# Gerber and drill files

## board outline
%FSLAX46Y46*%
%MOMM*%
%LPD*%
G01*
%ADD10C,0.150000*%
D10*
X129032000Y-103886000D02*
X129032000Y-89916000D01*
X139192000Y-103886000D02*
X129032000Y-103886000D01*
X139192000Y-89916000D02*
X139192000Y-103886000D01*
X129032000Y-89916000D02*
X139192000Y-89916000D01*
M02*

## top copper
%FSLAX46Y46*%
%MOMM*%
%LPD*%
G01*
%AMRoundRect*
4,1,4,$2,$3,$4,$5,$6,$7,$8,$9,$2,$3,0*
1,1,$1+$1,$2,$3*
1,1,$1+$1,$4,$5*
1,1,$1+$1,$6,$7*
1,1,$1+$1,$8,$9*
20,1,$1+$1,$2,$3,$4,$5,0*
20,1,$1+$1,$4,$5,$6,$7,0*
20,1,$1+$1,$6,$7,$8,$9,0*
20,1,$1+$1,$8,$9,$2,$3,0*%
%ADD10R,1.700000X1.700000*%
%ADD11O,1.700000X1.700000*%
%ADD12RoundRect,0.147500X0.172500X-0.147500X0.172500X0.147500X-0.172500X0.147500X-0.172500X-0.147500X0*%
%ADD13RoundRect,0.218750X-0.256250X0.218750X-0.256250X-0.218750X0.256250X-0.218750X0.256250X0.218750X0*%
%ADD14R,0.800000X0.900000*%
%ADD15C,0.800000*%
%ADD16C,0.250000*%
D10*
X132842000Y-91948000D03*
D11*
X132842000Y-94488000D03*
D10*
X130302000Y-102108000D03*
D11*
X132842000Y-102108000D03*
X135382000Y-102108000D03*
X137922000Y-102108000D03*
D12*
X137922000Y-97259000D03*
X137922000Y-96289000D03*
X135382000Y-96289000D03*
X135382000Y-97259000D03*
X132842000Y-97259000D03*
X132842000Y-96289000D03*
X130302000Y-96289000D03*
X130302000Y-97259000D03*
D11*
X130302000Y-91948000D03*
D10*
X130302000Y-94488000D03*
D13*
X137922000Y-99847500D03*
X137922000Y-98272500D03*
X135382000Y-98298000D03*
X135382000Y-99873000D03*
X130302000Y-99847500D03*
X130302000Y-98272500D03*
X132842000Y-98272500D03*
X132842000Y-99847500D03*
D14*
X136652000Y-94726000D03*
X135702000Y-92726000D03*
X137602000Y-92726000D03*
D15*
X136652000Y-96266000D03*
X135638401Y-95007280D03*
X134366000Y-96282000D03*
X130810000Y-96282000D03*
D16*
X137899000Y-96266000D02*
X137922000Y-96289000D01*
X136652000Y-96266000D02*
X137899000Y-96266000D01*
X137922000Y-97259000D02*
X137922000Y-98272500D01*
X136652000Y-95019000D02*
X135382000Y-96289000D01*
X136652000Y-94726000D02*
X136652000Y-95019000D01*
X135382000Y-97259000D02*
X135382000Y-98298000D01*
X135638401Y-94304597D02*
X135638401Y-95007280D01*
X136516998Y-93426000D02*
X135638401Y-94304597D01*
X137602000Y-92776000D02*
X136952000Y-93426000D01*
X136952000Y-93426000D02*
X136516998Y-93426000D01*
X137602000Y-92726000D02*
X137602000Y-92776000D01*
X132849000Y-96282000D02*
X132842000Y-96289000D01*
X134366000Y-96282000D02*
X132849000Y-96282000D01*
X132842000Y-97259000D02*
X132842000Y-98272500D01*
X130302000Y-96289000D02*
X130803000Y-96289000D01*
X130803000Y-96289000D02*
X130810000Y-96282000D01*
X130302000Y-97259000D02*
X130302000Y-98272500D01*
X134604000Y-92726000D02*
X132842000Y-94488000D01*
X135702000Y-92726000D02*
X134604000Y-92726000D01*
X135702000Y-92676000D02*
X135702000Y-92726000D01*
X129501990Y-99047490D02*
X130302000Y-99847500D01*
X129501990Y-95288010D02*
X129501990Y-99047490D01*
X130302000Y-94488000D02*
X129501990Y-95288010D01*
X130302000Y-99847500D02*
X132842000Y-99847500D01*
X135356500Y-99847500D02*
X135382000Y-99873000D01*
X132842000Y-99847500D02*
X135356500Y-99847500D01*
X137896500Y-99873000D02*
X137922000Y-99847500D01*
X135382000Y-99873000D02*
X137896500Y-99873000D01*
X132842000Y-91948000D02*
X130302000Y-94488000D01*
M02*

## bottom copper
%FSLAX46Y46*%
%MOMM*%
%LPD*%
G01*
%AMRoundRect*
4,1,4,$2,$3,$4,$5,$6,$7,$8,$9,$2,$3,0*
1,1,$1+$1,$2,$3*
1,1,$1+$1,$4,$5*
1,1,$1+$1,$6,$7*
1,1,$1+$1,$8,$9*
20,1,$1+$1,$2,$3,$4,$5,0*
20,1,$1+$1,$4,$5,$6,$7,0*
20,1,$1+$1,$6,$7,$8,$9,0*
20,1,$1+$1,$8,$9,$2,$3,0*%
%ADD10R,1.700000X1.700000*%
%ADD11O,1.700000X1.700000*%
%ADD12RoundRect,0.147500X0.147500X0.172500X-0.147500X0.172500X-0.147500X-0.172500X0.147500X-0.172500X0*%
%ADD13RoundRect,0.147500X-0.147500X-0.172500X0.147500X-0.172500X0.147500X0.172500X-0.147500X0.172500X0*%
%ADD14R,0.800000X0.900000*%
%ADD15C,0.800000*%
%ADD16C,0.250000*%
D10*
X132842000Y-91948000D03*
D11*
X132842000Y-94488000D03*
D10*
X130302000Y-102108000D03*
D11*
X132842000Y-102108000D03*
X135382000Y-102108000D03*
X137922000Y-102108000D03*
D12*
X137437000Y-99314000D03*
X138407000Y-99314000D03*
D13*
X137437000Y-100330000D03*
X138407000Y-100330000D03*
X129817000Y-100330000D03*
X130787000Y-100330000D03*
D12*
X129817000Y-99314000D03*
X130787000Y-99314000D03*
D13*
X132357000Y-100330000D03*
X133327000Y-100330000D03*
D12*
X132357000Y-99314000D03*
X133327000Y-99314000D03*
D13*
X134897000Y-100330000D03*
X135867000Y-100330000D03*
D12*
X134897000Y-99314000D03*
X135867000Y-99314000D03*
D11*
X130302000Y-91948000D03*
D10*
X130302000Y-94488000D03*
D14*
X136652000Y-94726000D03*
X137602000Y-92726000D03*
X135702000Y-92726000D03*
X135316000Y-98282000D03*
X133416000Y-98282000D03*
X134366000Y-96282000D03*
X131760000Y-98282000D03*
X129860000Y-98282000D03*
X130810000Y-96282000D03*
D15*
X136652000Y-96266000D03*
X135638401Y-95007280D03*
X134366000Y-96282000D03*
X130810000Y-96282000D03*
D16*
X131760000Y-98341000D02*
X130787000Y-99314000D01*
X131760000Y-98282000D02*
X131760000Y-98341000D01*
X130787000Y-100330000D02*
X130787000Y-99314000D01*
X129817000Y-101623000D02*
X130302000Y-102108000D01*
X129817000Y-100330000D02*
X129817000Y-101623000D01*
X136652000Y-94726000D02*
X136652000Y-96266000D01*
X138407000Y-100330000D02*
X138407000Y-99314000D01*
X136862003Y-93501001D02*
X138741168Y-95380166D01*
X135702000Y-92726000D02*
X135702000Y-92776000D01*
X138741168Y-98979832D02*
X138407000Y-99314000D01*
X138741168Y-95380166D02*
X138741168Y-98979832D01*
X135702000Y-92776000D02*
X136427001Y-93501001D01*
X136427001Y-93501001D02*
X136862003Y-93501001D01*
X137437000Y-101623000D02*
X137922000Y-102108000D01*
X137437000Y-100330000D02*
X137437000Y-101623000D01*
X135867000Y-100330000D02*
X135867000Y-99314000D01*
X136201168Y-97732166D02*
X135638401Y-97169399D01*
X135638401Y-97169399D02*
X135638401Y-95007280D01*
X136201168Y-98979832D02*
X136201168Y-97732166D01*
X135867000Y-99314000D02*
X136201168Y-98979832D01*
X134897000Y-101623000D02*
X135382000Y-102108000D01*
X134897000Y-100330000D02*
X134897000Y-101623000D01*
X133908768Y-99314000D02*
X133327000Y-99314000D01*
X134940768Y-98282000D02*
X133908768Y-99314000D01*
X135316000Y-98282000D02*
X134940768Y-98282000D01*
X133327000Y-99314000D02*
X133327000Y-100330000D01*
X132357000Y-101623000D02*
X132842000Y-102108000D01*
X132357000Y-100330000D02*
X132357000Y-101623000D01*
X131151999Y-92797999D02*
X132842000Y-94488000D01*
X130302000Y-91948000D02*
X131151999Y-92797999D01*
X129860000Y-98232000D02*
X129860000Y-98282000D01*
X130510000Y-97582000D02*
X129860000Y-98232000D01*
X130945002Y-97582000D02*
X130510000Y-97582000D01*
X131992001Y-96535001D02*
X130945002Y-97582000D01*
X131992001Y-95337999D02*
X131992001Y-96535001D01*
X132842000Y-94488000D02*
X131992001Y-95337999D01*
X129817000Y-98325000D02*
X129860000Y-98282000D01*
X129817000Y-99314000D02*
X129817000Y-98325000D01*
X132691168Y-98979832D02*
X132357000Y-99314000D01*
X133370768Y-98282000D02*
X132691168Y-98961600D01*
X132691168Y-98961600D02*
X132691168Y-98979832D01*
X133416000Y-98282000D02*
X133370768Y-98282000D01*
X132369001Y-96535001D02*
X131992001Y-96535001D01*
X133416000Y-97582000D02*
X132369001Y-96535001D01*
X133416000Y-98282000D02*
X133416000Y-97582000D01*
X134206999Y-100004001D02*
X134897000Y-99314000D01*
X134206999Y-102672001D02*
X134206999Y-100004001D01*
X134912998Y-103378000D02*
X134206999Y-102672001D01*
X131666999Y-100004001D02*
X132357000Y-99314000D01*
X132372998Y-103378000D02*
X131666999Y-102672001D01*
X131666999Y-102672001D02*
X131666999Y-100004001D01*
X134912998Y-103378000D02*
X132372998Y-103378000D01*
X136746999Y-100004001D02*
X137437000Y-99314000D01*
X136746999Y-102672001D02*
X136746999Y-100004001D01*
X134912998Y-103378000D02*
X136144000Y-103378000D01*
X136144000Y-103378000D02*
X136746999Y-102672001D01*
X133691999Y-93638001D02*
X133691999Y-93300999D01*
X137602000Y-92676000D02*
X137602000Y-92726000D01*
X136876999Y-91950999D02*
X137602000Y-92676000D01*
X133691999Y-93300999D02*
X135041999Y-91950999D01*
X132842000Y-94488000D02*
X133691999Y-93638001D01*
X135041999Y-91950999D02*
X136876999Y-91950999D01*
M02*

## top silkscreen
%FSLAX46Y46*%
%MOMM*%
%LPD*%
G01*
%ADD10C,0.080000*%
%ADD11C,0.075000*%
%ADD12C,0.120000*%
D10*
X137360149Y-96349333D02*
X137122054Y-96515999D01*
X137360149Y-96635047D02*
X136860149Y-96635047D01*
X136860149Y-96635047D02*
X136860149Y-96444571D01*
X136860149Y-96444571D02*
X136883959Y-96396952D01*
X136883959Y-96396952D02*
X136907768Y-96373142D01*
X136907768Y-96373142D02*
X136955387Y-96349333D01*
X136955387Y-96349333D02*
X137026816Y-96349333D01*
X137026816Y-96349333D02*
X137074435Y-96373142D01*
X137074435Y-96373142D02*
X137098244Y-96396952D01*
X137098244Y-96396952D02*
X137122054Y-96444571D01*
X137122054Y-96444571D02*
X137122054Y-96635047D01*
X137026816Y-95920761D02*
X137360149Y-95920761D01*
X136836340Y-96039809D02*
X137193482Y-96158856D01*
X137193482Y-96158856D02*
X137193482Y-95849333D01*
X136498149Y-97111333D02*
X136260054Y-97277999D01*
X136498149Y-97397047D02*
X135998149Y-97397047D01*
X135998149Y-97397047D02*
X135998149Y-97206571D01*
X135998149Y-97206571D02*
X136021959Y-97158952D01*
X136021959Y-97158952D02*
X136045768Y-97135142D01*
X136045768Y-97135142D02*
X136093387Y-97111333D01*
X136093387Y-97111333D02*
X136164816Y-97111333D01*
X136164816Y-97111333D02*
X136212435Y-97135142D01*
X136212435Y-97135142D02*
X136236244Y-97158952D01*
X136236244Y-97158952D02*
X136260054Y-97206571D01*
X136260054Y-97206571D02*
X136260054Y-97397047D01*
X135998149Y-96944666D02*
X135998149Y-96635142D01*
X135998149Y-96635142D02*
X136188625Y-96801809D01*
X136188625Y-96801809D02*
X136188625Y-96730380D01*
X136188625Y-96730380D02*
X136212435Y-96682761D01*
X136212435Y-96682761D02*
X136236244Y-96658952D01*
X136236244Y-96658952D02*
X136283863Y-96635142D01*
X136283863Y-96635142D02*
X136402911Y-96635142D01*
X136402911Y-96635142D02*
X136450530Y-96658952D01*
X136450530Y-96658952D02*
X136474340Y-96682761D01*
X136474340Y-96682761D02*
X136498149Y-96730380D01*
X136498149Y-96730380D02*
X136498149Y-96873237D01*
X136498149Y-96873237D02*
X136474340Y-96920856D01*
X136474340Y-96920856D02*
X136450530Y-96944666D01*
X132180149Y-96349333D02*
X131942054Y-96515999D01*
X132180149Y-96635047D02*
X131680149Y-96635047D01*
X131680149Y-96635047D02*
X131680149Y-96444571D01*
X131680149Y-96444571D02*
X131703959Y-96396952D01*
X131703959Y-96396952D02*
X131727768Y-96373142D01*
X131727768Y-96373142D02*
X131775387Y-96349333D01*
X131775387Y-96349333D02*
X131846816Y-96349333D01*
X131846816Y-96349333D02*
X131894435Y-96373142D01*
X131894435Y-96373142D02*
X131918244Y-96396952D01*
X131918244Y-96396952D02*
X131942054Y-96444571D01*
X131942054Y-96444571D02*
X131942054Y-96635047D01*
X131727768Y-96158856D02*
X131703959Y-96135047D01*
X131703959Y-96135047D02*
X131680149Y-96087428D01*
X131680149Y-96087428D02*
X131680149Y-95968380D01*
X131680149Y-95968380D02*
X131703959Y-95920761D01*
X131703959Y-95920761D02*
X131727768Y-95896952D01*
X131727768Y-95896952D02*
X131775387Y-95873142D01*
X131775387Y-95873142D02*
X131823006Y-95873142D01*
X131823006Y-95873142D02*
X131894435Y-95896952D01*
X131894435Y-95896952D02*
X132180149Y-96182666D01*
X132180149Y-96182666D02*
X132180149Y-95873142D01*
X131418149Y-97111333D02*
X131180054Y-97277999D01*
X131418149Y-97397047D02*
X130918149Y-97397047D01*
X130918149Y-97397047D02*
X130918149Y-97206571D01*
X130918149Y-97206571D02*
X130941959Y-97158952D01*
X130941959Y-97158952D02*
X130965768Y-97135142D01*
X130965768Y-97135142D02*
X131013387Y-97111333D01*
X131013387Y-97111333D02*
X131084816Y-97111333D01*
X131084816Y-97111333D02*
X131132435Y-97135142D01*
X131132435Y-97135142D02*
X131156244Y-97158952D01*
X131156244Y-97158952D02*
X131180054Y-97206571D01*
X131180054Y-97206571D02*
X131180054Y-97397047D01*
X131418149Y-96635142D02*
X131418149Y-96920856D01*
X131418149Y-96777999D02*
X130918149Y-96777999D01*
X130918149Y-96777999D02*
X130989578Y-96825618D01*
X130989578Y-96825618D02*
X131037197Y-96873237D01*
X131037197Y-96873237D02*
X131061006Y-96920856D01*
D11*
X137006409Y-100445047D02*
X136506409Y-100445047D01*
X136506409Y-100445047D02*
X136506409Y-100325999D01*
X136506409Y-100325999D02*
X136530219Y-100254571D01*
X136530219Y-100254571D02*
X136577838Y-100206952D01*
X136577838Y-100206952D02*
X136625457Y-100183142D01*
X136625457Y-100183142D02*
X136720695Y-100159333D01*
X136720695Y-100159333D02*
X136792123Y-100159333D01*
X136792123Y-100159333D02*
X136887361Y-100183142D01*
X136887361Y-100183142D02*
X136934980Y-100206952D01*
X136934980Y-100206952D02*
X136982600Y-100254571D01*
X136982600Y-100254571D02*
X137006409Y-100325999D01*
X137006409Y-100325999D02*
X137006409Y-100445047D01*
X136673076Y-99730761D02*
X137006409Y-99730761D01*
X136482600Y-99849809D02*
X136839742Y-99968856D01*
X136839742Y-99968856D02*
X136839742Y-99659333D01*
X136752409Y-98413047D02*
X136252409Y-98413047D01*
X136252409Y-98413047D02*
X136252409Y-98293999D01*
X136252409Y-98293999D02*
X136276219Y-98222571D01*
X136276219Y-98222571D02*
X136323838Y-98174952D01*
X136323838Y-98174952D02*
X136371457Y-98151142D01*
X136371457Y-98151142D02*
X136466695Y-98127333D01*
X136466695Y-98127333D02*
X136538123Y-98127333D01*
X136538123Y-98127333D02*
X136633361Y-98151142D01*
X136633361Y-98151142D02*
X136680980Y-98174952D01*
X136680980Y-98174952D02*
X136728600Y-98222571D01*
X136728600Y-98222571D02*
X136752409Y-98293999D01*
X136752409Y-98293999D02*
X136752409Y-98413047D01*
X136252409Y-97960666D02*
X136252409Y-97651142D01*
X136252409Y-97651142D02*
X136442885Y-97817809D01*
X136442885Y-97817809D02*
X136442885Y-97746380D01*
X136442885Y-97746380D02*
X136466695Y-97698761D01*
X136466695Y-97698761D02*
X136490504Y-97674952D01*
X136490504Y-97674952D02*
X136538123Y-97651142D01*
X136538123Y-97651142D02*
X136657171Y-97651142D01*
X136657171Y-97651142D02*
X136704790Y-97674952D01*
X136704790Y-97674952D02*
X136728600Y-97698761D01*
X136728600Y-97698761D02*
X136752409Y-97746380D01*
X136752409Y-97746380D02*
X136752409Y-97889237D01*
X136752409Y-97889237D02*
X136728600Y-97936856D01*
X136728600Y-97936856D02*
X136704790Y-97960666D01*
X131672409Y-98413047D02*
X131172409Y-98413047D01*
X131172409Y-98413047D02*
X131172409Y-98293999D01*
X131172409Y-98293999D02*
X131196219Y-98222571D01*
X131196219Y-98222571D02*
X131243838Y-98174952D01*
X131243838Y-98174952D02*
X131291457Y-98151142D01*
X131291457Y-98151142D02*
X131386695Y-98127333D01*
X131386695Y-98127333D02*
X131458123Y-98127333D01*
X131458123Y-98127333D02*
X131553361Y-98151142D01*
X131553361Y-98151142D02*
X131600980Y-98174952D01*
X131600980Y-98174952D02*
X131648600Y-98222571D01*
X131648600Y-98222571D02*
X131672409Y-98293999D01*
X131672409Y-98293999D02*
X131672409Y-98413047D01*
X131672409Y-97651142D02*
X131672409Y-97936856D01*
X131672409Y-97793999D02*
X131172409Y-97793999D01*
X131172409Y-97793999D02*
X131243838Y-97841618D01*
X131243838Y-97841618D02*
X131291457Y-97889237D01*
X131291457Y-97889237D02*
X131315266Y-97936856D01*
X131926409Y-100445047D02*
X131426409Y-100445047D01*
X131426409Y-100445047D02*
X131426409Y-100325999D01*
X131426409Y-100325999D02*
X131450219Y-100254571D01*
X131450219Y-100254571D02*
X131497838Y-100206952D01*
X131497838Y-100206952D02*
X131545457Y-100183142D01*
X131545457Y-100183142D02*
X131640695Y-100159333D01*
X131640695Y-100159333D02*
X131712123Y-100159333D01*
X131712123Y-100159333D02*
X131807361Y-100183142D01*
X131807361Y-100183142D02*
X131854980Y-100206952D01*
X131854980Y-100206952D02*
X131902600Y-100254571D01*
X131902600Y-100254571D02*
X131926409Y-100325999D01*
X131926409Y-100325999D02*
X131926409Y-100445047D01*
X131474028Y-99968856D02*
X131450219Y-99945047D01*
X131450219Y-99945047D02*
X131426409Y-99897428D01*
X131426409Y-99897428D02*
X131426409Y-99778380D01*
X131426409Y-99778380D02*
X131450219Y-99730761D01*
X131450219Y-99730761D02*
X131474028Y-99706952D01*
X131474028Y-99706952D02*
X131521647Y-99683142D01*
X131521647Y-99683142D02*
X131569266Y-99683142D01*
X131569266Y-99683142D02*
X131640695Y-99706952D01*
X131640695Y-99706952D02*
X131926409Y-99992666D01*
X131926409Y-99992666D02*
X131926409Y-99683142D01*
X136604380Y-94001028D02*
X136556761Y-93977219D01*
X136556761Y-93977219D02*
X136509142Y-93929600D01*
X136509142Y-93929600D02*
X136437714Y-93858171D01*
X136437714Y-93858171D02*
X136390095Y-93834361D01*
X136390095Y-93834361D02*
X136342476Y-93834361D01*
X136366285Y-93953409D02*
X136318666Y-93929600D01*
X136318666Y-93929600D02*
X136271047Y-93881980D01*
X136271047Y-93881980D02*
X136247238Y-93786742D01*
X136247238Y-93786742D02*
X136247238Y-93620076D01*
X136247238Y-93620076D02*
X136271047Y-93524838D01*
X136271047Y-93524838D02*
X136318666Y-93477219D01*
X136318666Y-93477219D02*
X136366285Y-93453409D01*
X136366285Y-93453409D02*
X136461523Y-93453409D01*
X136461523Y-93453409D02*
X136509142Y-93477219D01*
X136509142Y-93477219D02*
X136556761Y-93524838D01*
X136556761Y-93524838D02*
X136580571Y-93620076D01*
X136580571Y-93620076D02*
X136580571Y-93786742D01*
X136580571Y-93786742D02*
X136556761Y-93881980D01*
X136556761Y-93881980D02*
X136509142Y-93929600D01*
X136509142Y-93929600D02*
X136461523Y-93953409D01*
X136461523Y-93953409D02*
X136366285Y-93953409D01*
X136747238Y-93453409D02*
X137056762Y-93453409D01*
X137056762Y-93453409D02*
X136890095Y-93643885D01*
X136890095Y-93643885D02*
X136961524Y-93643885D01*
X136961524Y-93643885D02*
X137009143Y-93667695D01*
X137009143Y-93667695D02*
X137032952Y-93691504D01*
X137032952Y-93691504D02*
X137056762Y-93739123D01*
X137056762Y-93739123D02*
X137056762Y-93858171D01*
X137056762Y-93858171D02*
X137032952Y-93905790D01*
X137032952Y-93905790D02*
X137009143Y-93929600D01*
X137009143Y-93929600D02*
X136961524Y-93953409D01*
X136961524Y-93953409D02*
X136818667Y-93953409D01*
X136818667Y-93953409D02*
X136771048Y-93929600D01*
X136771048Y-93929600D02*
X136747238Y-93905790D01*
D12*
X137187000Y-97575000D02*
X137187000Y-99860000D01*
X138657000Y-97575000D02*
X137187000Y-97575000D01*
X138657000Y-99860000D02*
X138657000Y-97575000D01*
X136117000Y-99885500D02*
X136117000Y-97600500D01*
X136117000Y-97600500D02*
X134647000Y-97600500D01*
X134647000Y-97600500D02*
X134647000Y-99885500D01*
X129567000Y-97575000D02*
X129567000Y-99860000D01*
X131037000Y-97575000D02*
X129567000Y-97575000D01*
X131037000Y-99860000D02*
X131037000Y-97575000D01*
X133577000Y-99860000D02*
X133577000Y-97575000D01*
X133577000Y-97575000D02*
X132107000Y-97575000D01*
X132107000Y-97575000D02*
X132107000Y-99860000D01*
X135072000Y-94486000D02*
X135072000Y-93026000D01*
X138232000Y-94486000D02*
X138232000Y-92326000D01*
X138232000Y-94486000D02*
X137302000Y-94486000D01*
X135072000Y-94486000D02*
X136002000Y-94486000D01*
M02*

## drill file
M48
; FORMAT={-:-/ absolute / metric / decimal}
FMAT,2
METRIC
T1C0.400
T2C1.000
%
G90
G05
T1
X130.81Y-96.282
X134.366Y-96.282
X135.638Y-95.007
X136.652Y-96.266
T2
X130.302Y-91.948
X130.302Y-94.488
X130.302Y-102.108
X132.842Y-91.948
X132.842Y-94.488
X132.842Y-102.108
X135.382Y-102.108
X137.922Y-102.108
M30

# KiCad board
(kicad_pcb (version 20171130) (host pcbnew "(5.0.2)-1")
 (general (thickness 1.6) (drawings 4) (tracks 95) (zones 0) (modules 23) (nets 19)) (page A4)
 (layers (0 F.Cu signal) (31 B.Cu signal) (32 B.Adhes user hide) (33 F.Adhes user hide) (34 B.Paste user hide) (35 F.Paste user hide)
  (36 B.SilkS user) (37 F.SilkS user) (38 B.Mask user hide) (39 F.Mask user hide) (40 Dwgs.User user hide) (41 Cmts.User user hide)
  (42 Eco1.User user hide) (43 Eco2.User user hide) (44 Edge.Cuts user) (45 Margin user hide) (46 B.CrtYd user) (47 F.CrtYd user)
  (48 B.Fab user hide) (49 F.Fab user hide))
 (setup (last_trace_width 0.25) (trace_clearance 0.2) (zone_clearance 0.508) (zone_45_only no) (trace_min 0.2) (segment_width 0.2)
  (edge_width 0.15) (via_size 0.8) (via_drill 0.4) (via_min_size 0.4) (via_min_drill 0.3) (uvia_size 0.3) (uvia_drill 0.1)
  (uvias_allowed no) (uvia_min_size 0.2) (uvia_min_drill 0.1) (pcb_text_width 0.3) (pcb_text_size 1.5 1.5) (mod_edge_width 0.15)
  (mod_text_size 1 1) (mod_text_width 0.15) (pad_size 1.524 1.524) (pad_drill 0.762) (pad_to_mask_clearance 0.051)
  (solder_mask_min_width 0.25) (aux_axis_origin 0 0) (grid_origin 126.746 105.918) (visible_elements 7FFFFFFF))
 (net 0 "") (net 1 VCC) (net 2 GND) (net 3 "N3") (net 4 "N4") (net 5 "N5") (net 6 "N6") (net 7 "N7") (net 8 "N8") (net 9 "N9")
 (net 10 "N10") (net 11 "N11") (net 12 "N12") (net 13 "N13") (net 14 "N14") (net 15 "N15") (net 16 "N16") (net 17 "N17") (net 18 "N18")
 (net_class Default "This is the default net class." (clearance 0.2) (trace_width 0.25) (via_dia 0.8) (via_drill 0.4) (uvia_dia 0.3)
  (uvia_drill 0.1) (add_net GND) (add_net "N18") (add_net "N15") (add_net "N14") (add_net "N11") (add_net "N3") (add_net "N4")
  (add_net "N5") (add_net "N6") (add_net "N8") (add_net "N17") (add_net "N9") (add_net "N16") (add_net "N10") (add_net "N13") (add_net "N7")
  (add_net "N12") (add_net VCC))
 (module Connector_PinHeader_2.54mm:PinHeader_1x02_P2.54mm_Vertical (layer B.Cu) (at 132.842 91.948 180)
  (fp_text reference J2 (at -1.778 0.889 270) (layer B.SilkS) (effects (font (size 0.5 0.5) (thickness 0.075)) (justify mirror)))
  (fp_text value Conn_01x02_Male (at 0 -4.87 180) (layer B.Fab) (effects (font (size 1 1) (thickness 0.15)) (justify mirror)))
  (pad 1 thru_hole rect (at 0 0 180) (size 1.7 1.7) (drill 1) (layers *.Cu *.Mask) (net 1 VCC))
  (pad 2 thru_hole oval (at 0 -2.54 180) (size 1.7 1.7) (drill 1) (layers *.Cu *.Mask) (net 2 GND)))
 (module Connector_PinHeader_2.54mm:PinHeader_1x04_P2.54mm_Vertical (layer B.Cu) (at 130.302 102.108 270)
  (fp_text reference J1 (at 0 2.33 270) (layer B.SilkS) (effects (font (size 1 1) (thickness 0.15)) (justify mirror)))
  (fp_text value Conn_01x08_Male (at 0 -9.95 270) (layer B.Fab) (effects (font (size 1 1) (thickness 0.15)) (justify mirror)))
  (pad 1 thru_hole rect (at 0 0 270) (size 1.7 1.7) (drill 1) (layers *.Cu *.Mask) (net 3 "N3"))
  (pad 2 thru_hole oval (at 0 -2.54 270) (size 1.7 1.7) (drill 1) (layers *.Cu *.Mask) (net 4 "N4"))
  (pad 3 thru_hole oval (at 0 -5.08 270) (size 1.7 1.7) (drill 1) (layers *.Cu *.Mask) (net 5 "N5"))
  (pad 4 thru_hole oval (at 0 -7.62 270) (size 1.7 1.7) (drill 1) (layers *.Cu *.Mask) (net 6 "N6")))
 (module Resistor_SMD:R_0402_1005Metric (layer B.Cu) (at 137.922 99.314 180)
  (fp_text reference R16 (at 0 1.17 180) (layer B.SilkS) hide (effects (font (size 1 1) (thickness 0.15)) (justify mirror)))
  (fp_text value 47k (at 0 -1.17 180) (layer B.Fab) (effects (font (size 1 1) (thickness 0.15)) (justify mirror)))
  (pad 2 smd roundrect (at 0.485 0 180) (size 0.59 0.64) (layers B.Cu B.Paste B.Mask) (roundrect_rratio 0.25) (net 2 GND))
  (pad 1 smd roundrect (at -0.485 0 180) (size 0.59 0.64) (layers B.Cu B.Paste B.Mask) (roundrect_rratio 0.25) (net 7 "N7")))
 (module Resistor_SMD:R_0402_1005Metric (layer B.Cu) (at 137.922 100.33)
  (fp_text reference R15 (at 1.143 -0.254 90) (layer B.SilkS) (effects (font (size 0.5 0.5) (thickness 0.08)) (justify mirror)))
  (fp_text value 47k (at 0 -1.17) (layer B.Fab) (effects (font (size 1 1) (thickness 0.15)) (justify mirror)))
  (pad 1 smd roundrect (at -0.485 0) (size 0.59 0.64) (layers B.Cu B.Paste B.Mask) (roundrect_rratio 0.25) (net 6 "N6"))
  (pad 2 smd roundrect (at 0.485 0) (size 0.59 0.64) (layers B.Cu B.Paste B.Mask) (roundrect_rratio 0.25) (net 7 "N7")))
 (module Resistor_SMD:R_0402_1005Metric (layer B.Cu) (at 130.302 100.33)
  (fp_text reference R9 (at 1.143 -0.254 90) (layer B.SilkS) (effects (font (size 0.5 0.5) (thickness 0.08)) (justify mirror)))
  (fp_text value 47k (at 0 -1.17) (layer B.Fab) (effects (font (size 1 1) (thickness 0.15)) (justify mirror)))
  (pad 1 smd roundrect (at -0.485 0) (size 0.59 0.64) (layers B.Cu B.Paste B.Mask) (roundrect_rratio 0.25) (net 3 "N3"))
  (pad 2 smd roundrect (at 0.485 0) (size 0.59 0.64) (layers B.Cu B.Paste B.Mask) (roundrect_rratio 0.25) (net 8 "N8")))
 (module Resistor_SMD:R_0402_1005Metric (layer B.Cu) (at 130.302 99.314 180)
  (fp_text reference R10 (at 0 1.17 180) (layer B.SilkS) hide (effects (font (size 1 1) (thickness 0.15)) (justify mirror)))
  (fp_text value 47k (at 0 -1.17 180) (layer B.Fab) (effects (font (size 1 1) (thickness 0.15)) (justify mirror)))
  (pad 2 smd roundrect (at 0.485 0 180) (size 0.59 0.64) (layers B.Cu B.Paste B.Mask) (roundrect_rratio 0.25) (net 2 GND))
  (pad 1 smd roundrect (at -0.485 0 180) (size 0.59 0.64) (layers B.Cu B.Paste B.Mask) (roundrect_rratio 0.25) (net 8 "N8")))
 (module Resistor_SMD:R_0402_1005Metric (layer B.Cu) (at 132.842 100.33)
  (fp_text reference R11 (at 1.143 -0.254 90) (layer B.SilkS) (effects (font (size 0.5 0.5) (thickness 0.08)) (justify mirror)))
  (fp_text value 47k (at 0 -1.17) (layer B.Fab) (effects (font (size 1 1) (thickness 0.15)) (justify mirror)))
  (pad 1 smd roundrect (at -0.485 0) (size 0.59 0.64) (layers B.Cu B.Paste B.Mask) (roundrect_rratio 0.25) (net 4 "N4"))
  (pad 2 smd roundrect (at 0.485 0) (size 0.59 0.64) (layers B.Cu B.Paste B.Mask) (roundrect_rratio 0.25) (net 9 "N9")))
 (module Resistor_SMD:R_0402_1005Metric (layer B.Cu) (at 132.842 99.314 180)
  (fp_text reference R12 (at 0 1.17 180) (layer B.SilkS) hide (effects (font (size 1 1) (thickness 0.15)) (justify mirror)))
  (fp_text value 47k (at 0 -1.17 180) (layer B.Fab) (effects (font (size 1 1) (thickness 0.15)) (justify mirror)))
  (pad 2 smd roundrect (at 0.485 0 180) (size 0.59 0.64) (layers B.Cu B.Paste B.Mask) (roundrect_rratio 0.25) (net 2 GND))
  (pad 1 smd roundrect (at -0.485 0 180) (size 0.59 0.64) (layers B.Cu B.Paste B.Mask) (roundrect_rratio 0.25) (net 9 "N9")))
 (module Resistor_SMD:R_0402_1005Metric (layer B.Cu) (at 135.382 100.33)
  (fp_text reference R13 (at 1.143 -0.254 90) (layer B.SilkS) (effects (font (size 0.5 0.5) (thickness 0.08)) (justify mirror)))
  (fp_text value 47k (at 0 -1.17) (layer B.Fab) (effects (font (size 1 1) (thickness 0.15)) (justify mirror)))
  (pad 1 smd roundrect (at -0.485 0) (size 0.59 0.64) (layers B.Cu B.Paste B.Mask) (roundrect_rratio 0.25) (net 5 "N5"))
  (pad 2 smd roundrect (at 0.485 0) (size 0.59 0.64) (layers B.Cu B.Paste B.Mask) (roundrect_rratio 0.25) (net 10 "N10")))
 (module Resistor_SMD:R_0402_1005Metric (layer B.Cu) (at 135.382 99.314 180)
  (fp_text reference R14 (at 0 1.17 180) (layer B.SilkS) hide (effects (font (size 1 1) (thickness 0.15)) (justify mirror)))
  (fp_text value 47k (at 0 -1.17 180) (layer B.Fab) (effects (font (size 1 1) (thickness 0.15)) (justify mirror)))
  (pad 2 smd roundrect (at 0.485 0 180) (size 0.59 0.64) (layers B.Cu B.Paste B.Mask) (roundrect_rratio 0.25) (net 2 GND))
  (pad 1 smd roundrect (at -0.485 0 180) (size 0.59 0.64) (layers B.Cu B.Paste B.Mask) (roundrect_rratio 0.25) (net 10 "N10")))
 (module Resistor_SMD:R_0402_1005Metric (layer F.Cu) (at 137.922 96.774 90)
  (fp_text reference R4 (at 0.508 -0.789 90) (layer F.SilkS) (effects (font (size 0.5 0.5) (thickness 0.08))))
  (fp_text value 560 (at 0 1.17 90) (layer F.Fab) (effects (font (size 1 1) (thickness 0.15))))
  (pad 1 smd roundrect (at -0.485 0 90) (size 0.59 0.64) (layers F.Cu F.Paste F.Mask) (roundrect_rratio 0.25) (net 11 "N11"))
  (pad 2 smd roundrect (at 0.485 0 90) (size 0.59 0.64) (layers F.Cu F.Paste F.Mask) (roundrect_rratio 0.25) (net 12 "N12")))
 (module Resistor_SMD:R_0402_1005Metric (layer F.Cu) (at 135.382 96.774 90)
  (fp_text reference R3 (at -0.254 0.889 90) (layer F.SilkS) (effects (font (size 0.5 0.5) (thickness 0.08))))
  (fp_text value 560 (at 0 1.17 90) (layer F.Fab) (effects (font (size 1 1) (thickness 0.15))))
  (pad 2 smd roundrect (at 0.485 0 90) (size 0.59 0.64) (layers F.Cu F.Paste F.Mask) (roundrect_rratio 0.25) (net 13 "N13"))
  (pad 1 smd roundrect (at -0.485 0 90) (size 0.59 0.64) (layers F.Cu F.Paste F.Mask) (roundrect_rratio 0.25) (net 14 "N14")))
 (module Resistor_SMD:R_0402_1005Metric (layer F.Cu) (at 132.842 96.774 90)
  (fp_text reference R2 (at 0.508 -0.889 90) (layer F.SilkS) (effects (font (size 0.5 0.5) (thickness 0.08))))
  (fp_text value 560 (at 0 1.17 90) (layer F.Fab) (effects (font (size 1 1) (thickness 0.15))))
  (pad 1 smd roundrect (at -0.485 0 90) (size 0.59 0.64) (layers F.Cu F.Paste F.Mask) (roundrect_rratio 0.25) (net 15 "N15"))
  (pad 2 smd roundrect (at 0.485 0 90) (size 0.59 0.64) (layers F.Cu F.Paste F.Mask) (roundrect_rratio 0.25) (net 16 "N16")))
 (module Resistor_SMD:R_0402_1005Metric (layer F.Cu) (at 130.302 96.774 90)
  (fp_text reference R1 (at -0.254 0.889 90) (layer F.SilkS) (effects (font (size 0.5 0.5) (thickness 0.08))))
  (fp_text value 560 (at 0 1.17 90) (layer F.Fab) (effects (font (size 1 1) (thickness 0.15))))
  (pad 2 smd roundrect (at 0.485 0 90) (size 0.59 0.64) (layers F.Cu F.Paste F.Mask) (roundrect_rratio 0.25) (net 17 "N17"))
  (pad 1 smd roundrect (at -0.485 0 90) (size 0.59 0.64) (layers F.Cu F.Paste F.Mask) (roundrect_rratio 0.25) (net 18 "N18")))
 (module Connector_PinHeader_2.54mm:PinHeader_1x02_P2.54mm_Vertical (layer B.Cu) (at 130.302 94.488)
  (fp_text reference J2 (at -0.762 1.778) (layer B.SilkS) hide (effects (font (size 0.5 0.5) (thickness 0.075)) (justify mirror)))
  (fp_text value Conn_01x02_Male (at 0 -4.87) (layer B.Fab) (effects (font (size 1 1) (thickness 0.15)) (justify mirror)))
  (pad 2 thru_hole oval (at 0 -2.54) (size 1.7 1.7) (drill 1) (layers *.Cu *.Mask) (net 2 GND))
  (pad 1 thru_hole rect (at 0 0) (size 1.7 1.7) (drill 1) (layers *.Cu *.Mask) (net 1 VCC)))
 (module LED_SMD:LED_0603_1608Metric (layer F.Cu) (at 137.922 99.06 270)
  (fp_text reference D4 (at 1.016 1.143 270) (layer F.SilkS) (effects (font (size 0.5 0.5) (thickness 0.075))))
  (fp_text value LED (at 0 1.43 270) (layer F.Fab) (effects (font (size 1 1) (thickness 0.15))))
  (fp_line (start -1.485 0.735) (end 0.8 0.735) (layer F.SilkS) (width 0.12))
  (fp_line (start -1.485 -0.735) (end -1.485 0.735) (layer F.SilkS) (width 0.12))
  (fp_line (start 0.8 -0.735) (end -1.485 -0.735) (layer F.SilkS) (width 0.12))
  (pad 2 smd roundrect (at 0.7875 0 270) (size 0.875 0.95) (layers F.Cu F.Paste F.Mask) (roundrect_rratio 0.25) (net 1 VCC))
  (pad 1 smd roundrect (at -0.7875 0 270) (size 0.875 0.95) (layers F.Cu F.Paste F.Mask) (roundrect_rratio 0.25) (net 11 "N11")))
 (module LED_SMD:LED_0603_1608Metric (layer F.Cu) (at 135.382 99.0855 270)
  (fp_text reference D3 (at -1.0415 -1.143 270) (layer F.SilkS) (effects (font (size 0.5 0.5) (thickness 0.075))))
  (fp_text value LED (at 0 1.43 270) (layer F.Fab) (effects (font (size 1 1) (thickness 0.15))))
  (fp_line (start 0.8 -0.735) (end -1.485 -0.735) (layer F.SilkS) (width 0.12))
  (fp_line (start -1.485 -0.735) (end -1.485 0.735) (layer F.SilkS) (width 0.12))
  (fp_line (start -1.485 0.735) (end 0.8 0.735) (layer F.SilkS) (width 0.12))
  (pad 1 smd roundrect (at -0.7875 0 270) (size 0.875 0.95) (layers F.Cu F.Paste F.Mask) (roundrect_rratio 0.25) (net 14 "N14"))
  (pad 2 smd roundrect (at 0.7875 0 270) (size 0.875 0.95) (layers F.Cu F.Paste F.Mask) (roundrect_rratio 0.25) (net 1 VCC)))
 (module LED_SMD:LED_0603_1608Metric (layer F.Cu) (at 130.302 99.06 270)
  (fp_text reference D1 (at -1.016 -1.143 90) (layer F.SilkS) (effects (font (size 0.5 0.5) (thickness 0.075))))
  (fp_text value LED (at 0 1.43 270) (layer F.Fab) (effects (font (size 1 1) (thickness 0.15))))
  (fp_line (start -1.485 0.735) (end 0.8 0.735) (layer F.SilkS) (width 0.12))
  (fp_line (start -1.485 -0.735) (end -1.485 0.735) (layer F.SilkS) (width 0.12))
  (fp_line (start 0.8 -0.735) (end -1.485 -0.735) (layer F.SilkS) (width 0.12))
  (pad 2 smd roundrect (at 0.7875 0 270) (size 0.875 0.95) (layers F.Cu F.Paste F.Mask) (roundrect_rratio 0.25) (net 1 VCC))
  (pad 1 smd roundrect (at -0.7875 0 270) (size 0.875 0.95) (layers F.Cu F.Paste F.Mask) (roundrect_rratio 0.25) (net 18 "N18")))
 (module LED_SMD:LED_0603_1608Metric (layer F.Cu) (at 132.842 99.06 270)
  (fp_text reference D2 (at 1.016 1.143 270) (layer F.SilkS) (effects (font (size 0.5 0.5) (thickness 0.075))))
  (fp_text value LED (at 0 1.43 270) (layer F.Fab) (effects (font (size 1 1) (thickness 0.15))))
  (fp_line (start 0.8 -0.735) (end -1.485 -0.735) (layer F.SilkS) (width 0.12))
  (fp_line (start -1.485 -0.735) (end -1.485 0.735) (layer F.SilkS) (width 0.12))
  (fp_line (start -1.485 0.735) (end 0.8 0.735) (layer F.SilkS) (width 0.12))
  (pad 1 smd roundrect (at -0.7875 0 270) (size 0.875 0.95) (layers F.Cu F.Paste F.Mask) (roundrect_rratio 0.25) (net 15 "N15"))
  (pad 2 smd roundrect (at 0.7875 0 270) (size 0.875 0.95) (layers F.Cu F.Paste F.Mask) (roundrect_rratio 0.25) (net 1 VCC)))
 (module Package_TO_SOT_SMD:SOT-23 (layer B.Cu) (at 136.652 93.726 270)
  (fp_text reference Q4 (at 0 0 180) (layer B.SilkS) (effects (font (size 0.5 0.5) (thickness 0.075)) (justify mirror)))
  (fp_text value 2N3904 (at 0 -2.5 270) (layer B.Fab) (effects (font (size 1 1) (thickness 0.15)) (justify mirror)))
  (pad 3 smd rect (at 1 0 270) (size 0.9 0.8) (layers B.Cu B.Paste B.Mask) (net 12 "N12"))
  (pad 2 smd rect (at -1 -0.95 270) (size 0.9 0.8) (layers B.Cu B.Paste B.Mask) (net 2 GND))
  (pad 1 smd rect (at -1 0.95 270) (size 0.9 0.8) (layers B.Cu B.Paste B.Mask) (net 7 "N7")))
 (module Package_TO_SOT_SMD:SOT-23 (layer F.Cu) (at 136.652 93.726 270)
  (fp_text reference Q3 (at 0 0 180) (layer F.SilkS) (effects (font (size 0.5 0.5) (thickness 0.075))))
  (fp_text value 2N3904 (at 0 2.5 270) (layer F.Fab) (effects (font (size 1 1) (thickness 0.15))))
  (fp_line (start 0.76 1.58) (end -0.7 1.58) (layer F.SilkS) (width 0.12))
  (fp_line (start 0.76 -1.58) (end -1.4 -1.58) (layer F.SilkS) (width 0.12))
  (fp_line (start 0.76 -1.58) (end 0.76 -0.65) (layer F.SilkS) (width 0.12))
  (fp_line (start 0.76 1.58) (end 0.76 0.65) (layer F.SilkS) (width 0.12))
  (pad 3 smd rect (at 1 0 270) (size 0.9 0.8) (layers F.Cu F.Paste F.Mask) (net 13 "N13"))
  (pad 2 smd rect (at -1 0.95 270) (size 0.9 0.8) (layers F.Cu F.Paste F.Mask) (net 2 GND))
  (pad 1 smd rect (at -1 -0.95 270) (size 0.9 0.8) (layers F.Cu F.Paste F.Mask) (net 10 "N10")))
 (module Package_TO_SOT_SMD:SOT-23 (layer B.Cu) (at 134.366 97.282 90)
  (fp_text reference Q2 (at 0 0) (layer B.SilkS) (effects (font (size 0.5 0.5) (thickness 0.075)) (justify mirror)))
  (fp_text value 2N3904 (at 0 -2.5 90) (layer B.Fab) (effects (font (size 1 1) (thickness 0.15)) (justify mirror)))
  (pad 1 smd rect (at -1 0.95 90) (size 0.9 0.8) (layers B.Cu B.Paste B.Mask) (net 9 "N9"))
  (pad 2 smd rect (at -1 -0.95 90) (size 0.9 0.8) (layers B.Cu B.Paste B.Mask) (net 2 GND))
  (pad 3 smd rect (at 1 0 90) (size 0.9 0.8) (layers B.Cu B.Paste B.Mask) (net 16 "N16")))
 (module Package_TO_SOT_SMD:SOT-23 (layer B.Cu) (at 130.81 97.282 90)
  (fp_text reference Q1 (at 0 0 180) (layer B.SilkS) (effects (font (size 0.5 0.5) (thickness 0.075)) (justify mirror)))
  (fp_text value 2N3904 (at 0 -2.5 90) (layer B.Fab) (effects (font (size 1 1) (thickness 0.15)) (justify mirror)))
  (pad 1 smd rect (at -1 0.95 90) (size 0.9 0.8) (layers B.Cu B.Paste B.Mask) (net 8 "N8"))
  (pad 2 smd rect (at -1 -0.95 90) (size 0.9 0.8) (layers B.Cu B.Paste B.Mask) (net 2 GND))
  (pad 3 smd rect (at 1 0 90) (size 0.9 0.8) (layers B.Cu B.Paste B.Mask) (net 17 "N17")))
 (gr_line (start 129.032 103.886) (end 129.032 89.916) (layer Edge.Cuts) (width 0.15))
 (gr_line (start 139.192 103.886) (end 129.032 103.886) (layer Edge.Cuts) (width 0.15))
 (gr_line (start 139.192 89.916) (end 139.192 103.886) (layer Edge.Cuts) (width 0.15))
 (gr_line (start 129.032 89.916) (end 139.192 89.916) (layer Edge.Cuts) (width 0.15))
 (segment (start 131.76 98.341) (end 130.787 99.314) (width 0.25) (layer B.Cu) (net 8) (status 30))
 (segment (start 131.76 98.282) (end 131.76 98.341) (width 0.25) (layer B.Cu) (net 8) (status 30))
 (segment (start 130.787 100.33) (end 130.787 99.314) (width 0.25) (layer B.Cu) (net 8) (status 30))
 (segment (start 129.817 101.623) (end 130.302 102.108) (width 0.25) (layer B.Cu) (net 3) (status 30))
 (segment (start 129.817 100.33) (end 129.817 101.623) (width 0.25) (layer B.Cu) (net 3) (status 30))
 (via (at 136.652 96.266) (size 0.8) (drill 0.4) (layers F.Cu B.Cu) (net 12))
 (segment (start 137.899 96.266) (end 137.922 96.289) (width 0.25) (layer F.Cu) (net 12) (status 30))
 (segment (start 136.652 96.266) (end 137.899 96.266) (width 0.25) (layer F.Cu) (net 12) (status 20))
 (segment (start 136.652 94.726) (end 136.652 96.266) (width 0.25) (layer B.Cu) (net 12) (status 10))
 (segment (start 137.922 97.259) (end 137.922 98.2725) (width 0.25) (layer F.Cu) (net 11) (status 30))
 (segment (start 138.407 100.33) (end 138.407 99.314) (width 0.25) (layer B.Cu) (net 7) (status 30))
 (segment (start 136.862003 93.501001) (end 138.741168 95.380166) (width 0.25) (layer B.Cu) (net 7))
 (segment (start 135.702 92.726) (end 135.702 92.776) (width 0.25) (layer B.Cu) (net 7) (status 30))
 (segment (start 138.741168 98.979832) (end 138.407 99.314) (width 0.25) (layer B.Cu) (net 7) (status 20))
 (segment (start 138.741168 95.380166) (end 138.741168 98.979832) (width 0.25) (layer B.Cu) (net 7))
 (segment (start 135.702 92.776) (end 136.427001 93.501001) (width 0.25) (layer B.Cu) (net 7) (status 10))
 (segment (start 136.427001 93.501001) (end 136.862003 93.501001) (width 0.25) (layer B.Cu) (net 7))
 (segment (start 137.437 101.623) (end 137.922 102.108) (width 0.25) (layer B.Cu) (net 6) (status 30))
 (segment (start 137.437 100.33) (end 137.437 101.623) (width 0.25) (layer B.Cu) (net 6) (status 30))
 (segment (start 136.652 95.019) (end 135.382 96.289) (width 0.25) (layer F.Cu) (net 13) (status 30))
 (segment (start 136.652 94.726) (end 136.652 95.019) (width 0.25) (layer F.Cu) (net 13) (status 30))
 (segment (start 135.382 97.259) (end 135.382 98.298) (width 0.25) (layer F.Cu) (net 14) (status 30))
 (segment (start 135.867 100.33) (end 135.867 99.314) (width 0.25) (layer B.Cu) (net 10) (status 30))
 (segment (start 136.201168 97.732166) (end 135.638401 97.169399) (width 0.25) (layer B.Cu) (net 10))
 (segment (start 135.638401 94.304597) (end 135.638401 95.00728) (width 0.25) (layer F.Cu) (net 10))
 (via (at 135.638401 95.00728) (size 0.8) (drill 0.4) (layers F.Cu B.Cu) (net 10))
 (segment (start 136.516998 93.426) (end 135.638401 94.304597) (width 0.25) (layer F.Cu) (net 10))
 (segment (start 137.602 92.776) (end 136.952 93.426) (width 0.25) (layer F.Cu) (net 10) (status 10))
 (segment (start 135.638401 97.169399) (end 135.638401 95.00728) (width 0.25) (layer B.Cu) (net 10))
 (segment (start 136.201168 98.979832) (end 136.201168 97.732166) (width 0.25) (layer B.Cu) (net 10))
 (segment (start 136.952 93.426) (end 136.516998 93.426) (width 0.25) (layer F.Cu) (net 10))
 (segment (start 135.867 99.314) (end 136.201168 98.979832) (width 0.25) (layer B.Cu) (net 10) (status 10))
 (segment (start 137.602 92.726) (end 137.602 92.776) (width 0.25) (layer F.Cu) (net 10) (status 30))
 (segment (start 134.897 101.623) (end 135.382 102.108) (width 0.25) (layer B.Cu) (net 5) (status 30))
 (segment (start 134.897 100.33) (end 134.897 101.623) (width 0.25) (layer B.Cu) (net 5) (status 30))
 (via (at 134.366 96.282) (size 0.8) (drill 0.4) (layers F.Cu B.Cu) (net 16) (status 30))
 (segment (start 132.849 96.282) (end 132.842 96.289) (width 0.25) (layer F.Cu) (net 16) (status 30))
 (segment (start 134.366 96.282) (end 132.849 96.282) (width 0.25) (layer F.Cu) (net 16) (status 20))
 (segment (start 132.842 97.259) (end 132.842 98.2725) (width 0.25) (layer F.Cu) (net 15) (status 30))
 (segment (start 133.908768 99.314) (end 133.327 99.314) (width 0.25) (layer B.Cu) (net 9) (status 20))
 (segment (start 134.940768 98.282) (end 133.908768 99.314) (width 0.25) (layer B.Cu) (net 9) (status 10))
 (segment (start 135.316 98.282) (end 134.940768 98.282) (width 0.25) (layer B.Cu) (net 9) (status 30))
 (segment (start 133.327 99.314) (end 133.327 100.33) (width 0.25) (layer B.Cu) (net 9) (status 30))
 (segment (start 132.357 101.623) (end 132.842 102.108) (width 0.25) (layer B.Cu) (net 4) (status 30))
 (segment (start 132.357 100.33) (end 132.357 101.623) (width 0.25) (layer B.Cu) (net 4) (status 30))
 (via (at 130.81 96.282) (size 0.8) (drill 0.4) (layers F.Cu B.Cu) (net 17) (status 30))
 (segment (start 130.302 96.289) (end 130.803 96.289) (width 0.25) (layer F.Cu) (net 17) (status 10))
 (segment (start 130.803 96.289) (end 130.81 96.282) (width 0.25) (layer F.Cu) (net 17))
 (segment (start 130.302 97.259) (end 130.302 98.2725) (width 0.25) (layer F.Cu) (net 18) (status 30))
 (segment (start 134.604 92.726) (end 132.842 94.488) (width 0.25) (layer F.Cu) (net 2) (status 20))
 (segment (start 135.702 92.726) (end 134.604 92.726) (width 0.25) (layer F.Cu) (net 2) (status 10))
 (segment (start 131.151999 92.797999) (end 132.842 94.488) (width 0.25) (layer B.Cu) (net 2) (status 30))
 (segment (start 130.302 91.948) (end 131.151999 92.797999) (width 0.25) (layer B.Cu) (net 2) (status 30))
 (segment (start 129.86 98.232) (end 129.86 98.282) (width 0.25) (layer B.Cu) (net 2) (status 30))
 (segment (start 130.51 97.582) (end 129.86 98.232) (width 0.25) (layer B.Cu) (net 2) (status 20))
 (segment (start 130.945002 97.582) (end 130.51 97.582) (width 0.25) (layer B.Cu) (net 2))
 (segment (start 131.992001 96.535001) (end 130.945002 97.582) (width 0.25) (layer B.Cu) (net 2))
 (segment (start 131.992001 95.337999) (end 131.992001 96.535001) (width 0.25) (layer B.Cu) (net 2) (status 10))
 (segment (start 132.842 94.488) (end 131.992001 95.337999) (width 0.25) (layer B.Cu) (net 2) (status 30))
 (segment (start 129.817 98.325) (end 129.86 98.282) (width 0.25) (layer B.Cu) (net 2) (status 30))
 (segment (start 129.817 99.314) (end 129.817 98.325) (width 0.25) (layer B.Cu) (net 2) (status 30))
 (segment (start 132.691168 98.979832) (end 132.357 99.314) (width 0.25) (layer B.Cu) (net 2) (status 20))
 (segment (start 133.370768 98.282) (end 132.691168 98.9616) (width 0.25) (layer B.Cu) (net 2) (status 10))
 (segment (start 132.691168 98.9616) (end 132.691168 98.979832) (width 0.25) (layer B.Cu) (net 2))
 (segment (start 133.416 98.282) (end 133.370768 98.282) (width 0.25) (layer B.Cu) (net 2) (status 30))
 (segment (start 132.369001 96.535001) (end 131.992001 96.535001) (width 0.25) (layer B.Cu) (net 2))
 (segment (start 133.416 97.582) (end 132.369001 96.535001) (width 0.25) (layer B.Cu) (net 2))
 (segment (start 133.416 98.282) (end 133.416 97.582) (width 0.25) (layer B.Cu) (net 2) (status 10))
 (segment (start 134.206999 100.004001) (end 134.897 99.314) (width 0.25) (layer B.Cu) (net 2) (status 20))
 (segment (start 134.206999 102.672001) (end 134.206999 100.004001) (width 0.25) (layer B.Cu) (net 2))
 (segment (start 134.912998 103.378) (end 134.206999 102.672001) (width 0.25) (layer B.Cu) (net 2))
 (segment (start 131.666999 100.004001) (end 132.357 99.314) (width 0.25) (layer B.Cu) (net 2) (status 20))
 (segment (start 132.372998 103.378) (end 131.666999 102.672001) (width 0.25) (layer B.Cu) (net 2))
 (segment (start 131.666999 102.672001) (end 131.666999 100.004001) (width 0.25) (layer B.Cu) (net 2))
 (segment (start 134.912998 103.378) (end 132.372998 103.378) (width 0.25) (layer B.Cu) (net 2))
 (segment (start 135.702 92.676) (end 135.702 92.726) (width 0.25) (layer F.Cu) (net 2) (status 30))
 (segment (start 136.746999 100.004001) (end 137.437 99.314) (width 0.25) (layer B.Cu) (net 2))
 (segment (start 136.746999 102.672001) (end 136.746999 100.004001) (width 0.25) (layer B.Cu) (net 2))
 (segment (start 134.912998 103.378) (end 136.144 103.378) (width 0.25) (layer B.Cu) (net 2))
 (segment (start 136.144 103.378) (end 136.746999 102.672001) (width 0.25) (layer B.Cu) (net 2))
 (segment (start 133.691999 93.638001) (end 133.691999 93.300999) (width 0.25) (layer B.Cu) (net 2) (status 1000010))
 (segment (start 137.602 92.676) (end 137.602 92.726) (width 0.25) (layer B.Cu) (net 2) (status 1000030))
 (segment (start 136.876999 91.950999) (end 137.602 92.676) (width 0.25) (layer B.Cu) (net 2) (status 1000020))
 (segment (start 133.691999 93.300999) (end 135.041999 91.950999) (width 0.25) (layer B.Cu) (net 2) (status 1000000))
 (segment (start 132.842 94.488) (end 133.691999 93.638001) (width 0.25) (layer B.Cu) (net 2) (status 1000030))
 (segment (start 135.041999 91.950999) (end 136.876999 91.950999) (width 0.25) (layer B.Cu) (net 2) (status 1000000))
 (segment (start 129.50199 99.04749) (end 130.302 99.8475) (width 0.25) (layer F.Cu) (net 1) (status 20))
 (segment (start 129.50199 95.28801) (end 129.50199 99.04749) (width 0.25) (layer F.Cu) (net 1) (status 10))
 (segment (start 130.302 94.488) (end 129.50199 95.28801) (width 0.25) (layer F.Cu) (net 1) (status 30))
 (segment (start 130.302 99.8475) (end 132.842 99.8475) (width 0.25) (layer F.Cu) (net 1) (status 30))
 (segment (start 135.3565 99.8475) (end 135.382 99.873) (width 0.25) (layer F.Cu) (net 1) (status 30))
 (segment (start 132.842 99.8475) (end 135.3565 99.8475) (width 0.25) (layer F.Cu) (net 1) (status 30))
 (segment (start 137.8965 99.873) (end 137.922 99.8475) (width 0.25) (layer F.Cu) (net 1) (status 30))
 (segment (start 135.382 99.873) (end 137.8965 99.873) (width 0.25) (layer F.Cu) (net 1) (status 30))
 (segment (start 132.842 91.948) (end 130.302 94.488) (width 0.25) (layer F.Cu) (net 1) (status 30)))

